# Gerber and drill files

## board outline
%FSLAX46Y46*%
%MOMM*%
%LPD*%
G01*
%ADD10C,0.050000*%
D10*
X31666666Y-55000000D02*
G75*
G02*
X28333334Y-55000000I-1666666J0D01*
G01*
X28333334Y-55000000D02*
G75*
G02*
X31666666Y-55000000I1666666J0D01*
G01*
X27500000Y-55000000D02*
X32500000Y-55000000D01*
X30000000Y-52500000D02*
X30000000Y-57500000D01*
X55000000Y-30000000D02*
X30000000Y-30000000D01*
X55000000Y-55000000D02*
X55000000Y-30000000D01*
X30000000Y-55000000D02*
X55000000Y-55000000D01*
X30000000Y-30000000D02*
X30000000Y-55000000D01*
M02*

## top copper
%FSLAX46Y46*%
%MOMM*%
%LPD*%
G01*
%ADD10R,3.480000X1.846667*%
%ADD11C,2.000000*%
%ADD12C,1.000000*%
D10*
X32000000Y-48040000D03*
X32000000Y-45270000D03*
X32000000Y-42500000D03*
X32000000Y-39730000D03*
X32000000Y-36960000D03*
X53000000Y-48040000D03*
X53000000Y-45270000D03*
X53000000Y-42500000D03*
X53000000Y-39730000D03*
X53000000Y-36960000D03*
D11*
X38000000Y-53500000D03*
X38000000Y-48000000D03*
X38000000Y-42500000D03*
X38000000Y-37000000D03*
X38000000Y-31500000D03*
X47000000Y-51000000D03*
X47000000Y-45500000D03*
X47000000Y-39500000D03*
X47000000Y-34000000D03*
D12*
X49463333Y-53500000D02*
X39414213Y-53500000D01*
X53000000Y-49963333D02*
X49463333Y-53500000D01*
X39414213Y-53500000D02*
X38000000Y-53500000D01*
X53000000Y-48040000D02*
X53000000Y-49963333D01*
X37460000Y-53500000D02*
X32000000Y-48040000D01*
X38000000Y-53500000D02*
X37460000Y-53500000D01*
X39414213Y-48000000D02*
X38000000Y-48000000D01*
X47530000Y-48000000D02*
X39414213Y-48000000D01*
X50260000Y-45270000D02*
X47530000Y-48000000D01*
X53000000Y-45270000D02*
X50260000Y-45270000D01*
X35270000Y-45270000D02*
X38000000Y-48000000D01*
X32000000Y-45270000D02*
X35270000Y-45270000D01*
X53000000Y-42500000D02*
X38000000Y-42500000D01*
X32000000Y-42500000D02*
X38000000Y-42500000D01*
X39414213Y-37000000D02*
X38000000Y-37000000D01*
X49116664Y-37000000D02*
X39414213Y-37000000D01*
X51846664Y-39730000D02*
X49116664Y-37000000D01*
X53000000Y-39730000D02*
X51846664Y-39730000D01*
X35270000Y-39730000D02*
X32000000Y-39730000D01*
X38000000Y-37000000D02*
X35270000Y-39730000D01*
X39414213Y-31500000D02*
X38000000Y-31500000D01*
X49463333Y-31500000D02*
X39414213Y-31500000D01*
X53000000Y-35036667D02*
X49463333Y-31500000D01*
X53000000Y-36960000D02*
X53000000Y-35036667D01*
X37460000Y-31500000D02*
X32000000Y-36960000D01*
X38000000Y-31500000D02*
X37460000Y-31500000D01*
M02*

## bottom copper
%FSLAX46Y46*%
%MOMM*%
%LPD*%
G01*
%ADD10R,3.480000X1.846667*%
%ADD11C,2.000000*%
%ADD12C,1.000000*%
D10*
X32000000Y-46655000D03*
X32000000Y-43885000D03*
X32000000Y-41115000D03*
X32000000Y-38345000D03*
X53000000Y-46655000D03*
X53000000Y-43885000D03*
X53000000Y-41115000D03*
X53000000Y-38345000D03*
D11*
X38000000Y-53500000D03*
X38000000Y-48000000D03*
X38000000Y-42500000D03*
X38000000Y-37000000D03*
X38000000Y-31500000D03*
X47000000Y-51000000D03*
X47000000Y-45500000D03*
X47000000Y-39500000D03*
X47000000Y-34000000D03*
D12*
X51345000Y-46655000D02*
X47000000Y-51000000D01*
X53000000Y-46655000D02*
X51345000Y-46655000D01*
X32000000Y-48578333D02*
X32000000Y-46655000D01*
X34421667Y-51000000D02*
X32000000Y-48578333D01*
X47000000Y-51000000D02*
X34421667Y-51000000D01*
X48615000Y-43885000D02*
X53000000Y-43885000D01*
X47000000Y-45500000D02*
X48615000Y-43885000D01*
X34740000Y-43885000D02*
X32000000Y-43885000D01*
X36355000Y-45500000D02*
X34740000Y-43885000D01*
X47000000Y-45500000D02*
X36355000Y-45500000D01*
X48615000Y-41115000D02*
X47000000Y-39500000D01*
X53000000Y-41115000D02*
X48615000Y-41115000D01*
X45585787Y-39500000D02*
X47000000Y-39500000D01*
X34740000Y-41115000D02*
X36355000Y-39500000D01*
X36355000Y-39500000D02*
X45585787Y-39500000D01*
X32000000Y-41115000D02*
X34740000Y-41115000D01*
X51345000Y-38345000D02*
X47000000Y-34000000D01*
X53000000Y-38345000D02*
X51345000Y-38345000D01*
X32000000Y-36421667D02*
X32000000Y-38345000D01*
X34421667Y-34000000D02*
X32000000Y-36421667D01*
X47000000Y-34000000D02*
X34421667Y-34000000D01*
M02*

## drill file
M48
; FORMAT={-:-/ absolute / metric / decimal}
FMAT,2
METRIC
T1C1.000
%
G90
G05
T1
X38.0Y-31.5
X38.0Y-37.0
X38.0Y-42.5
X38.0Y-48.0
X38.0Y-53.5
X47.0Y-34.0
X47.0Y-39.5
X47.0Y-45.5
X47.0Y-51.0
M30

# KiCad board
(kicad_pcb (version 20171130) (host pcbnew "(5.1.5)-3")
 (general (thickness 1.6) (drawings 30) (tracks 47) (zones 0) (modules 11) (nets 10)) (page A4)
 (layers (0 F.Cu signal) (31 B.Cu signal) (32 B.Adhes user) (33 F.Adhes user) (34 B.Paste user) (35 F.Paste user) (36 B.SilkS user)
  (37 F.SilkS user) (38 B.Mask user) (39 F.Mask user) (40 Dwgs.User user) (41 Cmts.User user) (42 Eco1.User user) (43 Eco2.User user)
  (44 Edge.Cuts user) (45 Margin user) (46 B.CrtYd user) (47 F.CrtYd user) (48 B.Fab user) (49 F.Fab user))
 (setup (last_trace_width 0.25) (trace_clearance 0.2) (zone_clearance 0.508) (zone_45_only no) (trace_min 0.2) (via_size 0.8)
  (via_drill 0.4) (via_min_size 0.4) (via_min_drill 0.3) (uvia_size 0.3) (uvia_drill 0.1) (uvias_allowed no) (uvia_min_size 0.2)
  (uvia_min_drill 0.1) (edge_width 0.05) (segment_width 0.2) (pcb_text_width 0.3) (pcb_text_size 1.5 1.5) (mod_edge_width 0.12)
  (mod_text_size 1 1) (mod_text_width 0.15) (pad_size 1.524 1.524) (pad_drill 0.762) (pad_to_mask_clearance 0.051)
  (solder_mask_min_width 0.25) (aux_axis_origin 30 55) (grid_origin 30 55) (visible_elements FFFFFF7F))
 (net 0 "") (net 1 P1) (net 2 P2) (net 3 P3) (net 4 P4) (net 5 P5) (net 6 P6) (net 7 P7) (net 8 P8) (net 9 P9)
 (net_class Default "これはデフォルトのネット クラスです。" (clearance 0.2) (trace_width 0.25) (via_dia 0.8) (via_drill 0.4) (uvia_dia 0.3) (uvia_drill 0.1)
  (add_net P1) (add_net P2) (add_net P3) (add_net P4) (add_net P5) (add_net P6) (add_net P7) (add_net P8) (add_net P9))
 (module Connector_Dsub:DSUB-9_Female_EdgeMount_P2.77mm (layer F.Cu) (at 32 42.5 270)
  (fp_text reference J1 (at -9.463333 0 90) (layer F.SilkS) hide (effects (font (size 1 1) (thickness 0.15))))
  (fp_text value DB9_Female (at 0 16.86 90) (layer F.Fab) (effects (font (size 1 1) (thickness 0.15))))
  (pad 1 smd rect (at 5.54 0 270) (size 1.846667 3.48) (layers F.Cu F.Paste F.Mask) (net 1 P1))
  (pad 2 smd rect (at 2.77 0 270) (size 1.846667 3.48) (layers F.Cu F.Paste F.Mask) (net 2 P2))
  (pad 3 smd rect (at 0 0 270) (size 1.846667 3.48) (layers F.Cu F.Paste F.Mask) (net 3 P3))
  (pad 4 smd rect (at -2.77 0 270) (size 1.846667 3.48) (layers F.Cu F.Paste F.Mask) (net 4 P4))
  (pad 5 smd rect (at -5.54 0 270) (size 1.846667 3.48) (layers F.Cu F.Paste F.Mask) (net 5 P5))
  (pad 6 smd rect (at 4.155 0 270) (size 1.846667 3.48) (layers B.Cu B.Paste B.Mask) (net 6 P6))
  (pad 7 smd rect (at 1.385 0 270) (size 1.846667 3.48) (layers B.Cu B.Paste B.Mask) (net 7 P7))
  (pad 8 smd rect (at -1.385 0 270) (size 1.846667 3.48) (layers B.Cu B.Paste B.Mask) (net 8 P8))
  (pad 9 smd rect (at -4.155 0 270) (size 1.846667 3.48) (layers B.Cu B.Paste B.Mask) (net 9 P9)))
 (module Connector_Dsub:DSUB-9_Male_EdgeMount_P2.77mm (layer F.Cu) (at 53 42.5 90)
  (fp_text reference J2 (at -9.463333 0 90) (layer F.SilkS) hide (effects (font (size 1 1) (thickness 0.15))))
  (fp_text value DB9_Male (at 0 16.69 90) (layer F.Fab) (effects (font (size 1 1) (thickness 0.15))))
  (pad 1 smd rect (at -5.54 0 90) (size 1.846667 3.48) (layers F.Cu F.Paste F.Mask) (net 1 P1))
  (pad 2 smd rect (at -2.77 0 90) (size 1.846667 3.48) (layers F.Cu F.Paste F.Mask) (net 2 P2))
  (pad 3 smd rect (at 0 0 90) (size 1.846667 3.48) (layers F.Cu F.Paste F.Mask) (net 3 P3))
  (pad 4 smd rect (at 2.77 0 90) (size 1.846667 3.48) (layers F.Cu F.Paste F.Mask) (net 4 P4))
  (pad 5 smd rect (at 5.54 0 90) (size 1.846667 3.48) (layers F.Cu F.Paste F.Mask) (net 5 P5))
  (pad 6 smd rect (at -4.155 0 90) (size 1.846667 3.48) (layers B.Cu B.Paste B.Mask) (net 6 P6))
  (pad 7 smd rect (at -1.385 0 90) (size 1.846667 3.48) (layers B.Cu B.Paste B.Mask) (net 7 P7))
  (pad 8 smd rect (at 1.385 0 90) (size 1.846667 3.48) (layers B.Cu B.Paste B.Mask) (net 8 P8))
  (pad 9 smd rect (at 4.155 0 90) (size 1.846667 3.48) (layers B.Cu B.Paste B.Mask) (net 9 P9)))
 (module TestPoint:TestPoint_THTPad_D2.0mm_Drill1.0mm (layer F.Cu) (at 38 53.5)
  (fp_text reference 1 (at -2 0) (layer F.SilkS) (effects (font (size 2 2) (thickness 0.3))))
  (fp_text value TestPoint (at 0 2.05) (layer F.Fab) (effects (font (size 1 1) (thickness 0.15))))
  (pad 1 thru_hole circle (at 0 0) (size 2 2) (drill 1) (layers *.Cu *.Mask) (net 1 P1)))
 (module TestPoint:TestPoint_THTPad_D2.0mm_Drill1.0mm (layer F.Cu) (at 38 48)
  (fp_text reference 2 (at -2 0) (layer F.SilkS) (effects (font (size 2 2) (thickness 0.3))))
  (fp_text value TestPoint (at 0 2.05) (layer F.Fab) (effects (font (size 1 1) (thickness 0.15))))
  (pad 1 thru_hole circle (at 0 0) (size 2 2) (drill 1) (layers *.Cu *.Mask) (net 2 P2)))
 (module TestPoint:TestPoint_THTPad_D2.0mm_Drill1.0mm (layer F.Cu) (at 38 42.5)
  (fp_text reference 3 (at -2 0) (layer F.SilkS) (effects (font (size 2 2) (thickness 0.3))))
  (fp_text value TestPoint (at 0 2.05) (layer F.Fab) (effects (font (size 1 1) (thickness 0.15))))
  (pad 1 thru_hole circle (at 0 0) (size 2 2) (drill 1) (layers *.Cu *.Mask) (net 3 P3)))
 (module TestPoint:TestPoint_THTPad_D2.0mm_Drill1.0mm (layer F.Cu) (at 38 37)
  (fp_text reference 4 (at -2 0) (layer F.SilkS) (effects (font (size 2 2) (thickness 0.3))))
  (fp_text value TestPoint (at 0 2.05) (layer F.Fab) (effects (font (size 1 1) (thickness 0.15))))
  (pad 1 thru_hole circle (at 0 0) (size 2 2) (drill 1) (layers *.Cu *.Mask) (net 4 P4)))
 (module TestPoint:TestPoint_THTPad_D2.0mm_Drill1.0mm (layer F.Cu) (at 38 31.5)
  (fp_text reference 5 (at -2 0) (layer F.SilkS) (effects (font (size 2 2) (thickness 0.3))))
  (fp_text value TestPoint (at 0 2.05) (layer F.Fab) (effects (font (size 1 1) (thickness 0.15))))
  (pad 1 thru_hole circle (at 0 0) (size 2 2) (drill 1) (layers *.Cu *.Mask) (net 5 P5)))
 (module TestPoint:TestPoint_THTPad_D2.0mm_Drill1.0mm (layer F.Cu) (at 47 51)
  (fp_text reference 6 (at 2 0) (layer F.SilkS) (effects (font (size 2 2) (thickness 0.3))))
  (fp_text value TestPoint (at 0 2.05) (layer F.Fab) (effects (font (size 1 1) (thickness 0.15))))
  (pad 1 thru_hole circle (at 0 0) (size 2 2) (drill 1) (layers *.Cu *.Mask) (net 6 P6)))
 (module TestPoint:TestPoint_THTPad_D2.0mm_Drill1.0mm (layer F.Cu) (at 47 45.5)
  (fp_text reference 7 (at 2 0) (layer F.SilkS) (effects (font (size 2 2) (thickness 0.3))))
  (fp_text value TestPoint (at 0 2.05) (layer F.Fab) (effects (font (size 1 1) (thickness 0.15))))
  (pad 1 thru_hole circle (at 0 0) (size 2 2) (drill 1) (layers *.Cu *.Mask) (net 7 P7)))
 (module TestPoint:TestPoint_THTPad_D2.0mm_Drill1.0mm (layer F.Cu) (at 47 39.5)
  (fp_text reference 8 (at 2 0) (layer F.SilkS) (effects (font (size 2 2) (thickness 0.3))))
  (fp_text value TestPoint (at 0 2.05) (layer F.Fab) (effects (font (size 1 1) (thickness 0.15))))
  (pad 1 thru_hole circle (at 0 0) (size 2 2) (drill 1) (layers *.Cu *.Mask) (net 8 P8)))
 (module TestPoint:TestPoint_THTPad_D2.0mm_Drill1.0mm (layer F.Cu) (at 47 34)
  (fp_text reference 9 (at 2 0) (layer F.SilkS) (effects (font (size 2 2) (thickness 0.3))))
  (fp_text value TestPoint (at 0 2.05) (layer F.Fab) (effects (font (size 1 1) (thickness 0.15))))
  (pad 1 thru_hole circle (at 0 0) (size 2 2) (drill 1) (layers *.Cu *.Mask) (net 9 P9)))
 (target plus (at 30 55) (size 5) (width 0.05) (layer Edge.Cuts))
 (gr_line (start 55 30) (end 30 30) (layer Edge.Cuts) (width 0.05))
 (gr_line (start 55 55) (end 55 30) (layer Edge.Cuts) (width 0.05))
 (gr_line (start 30 55) (end 55 55) (layer Edge.Cuts) (width 0.05))
 (gr_line (start 30 30) (end 30 55) (layer Edge.Cuts) (width 0.05))
 (segment (start 49.463333 53.5) (end 39.414213 53.5) (width 1) (layer F.Cu) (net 1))
 (segment (start 53 49.963333) (end 49.463333 53.5) (width 1) (layer F.Cu) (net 1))
 (segment (start 39.414213 53.5) (end 38 53.5) (width 1) (layer F.Cu) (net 1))
 (segment (start 53 48.04) (end 53 49.963333) (width 1) (layer F.Cu) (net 1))
 (segment (start 37.46 53.5) (end 32 48.04) (width 1) (layer F.Cu) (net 1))
 (segment (start 38 53.5) (end 37.46 53.5) (width 1) (layer F.Cu) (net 1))
 (segment (start 39.414213 48) (end 38 48) (width 1) (layer F.Cu) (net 2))
 (segment (start 47.53 48) (end 39.414213 48) (width 1) (layer F.Cu) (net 2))
 (segment (start 50.26 45.27) (end 47.53 48) (width 1) (layer F.Cu) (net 2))
 (segment (start 53 45.27) (end 50.26 45.27) (width 1) (layer F.Cu) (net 2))
 (segment (start 35.27 45.27) (end 38 48) (width 1) (layer F.Cu) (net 2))
 (segment (start 32 45.27) (end 35.27 45.27) (width 1) (layer F.Cu) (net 2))
 (segment (start 53 42.5) (end 38 42.5) (width 1) (layer F.Cu) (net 3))
 (segment (start 32 42.5) (end 38 42.5) (width 1) (layer F.Cu) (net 3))
 (segment (start 39.414213 37) (end 38 37) (width 1) (layer F.Cu) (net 4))
 (segment (start 49.116664 37) (end 39.414213 37) (width 1) (layer F.Cu) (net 4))
 (segment (start 51.846664 39.73) (end 49.116664 37) (width 1) (layer F.Cu) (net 4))
 (segment (start 53 39.73) (end 51.846664 39.73) (width 1) (layer F.Cu) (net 4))
 (segment (start 35.27 39.73) (end 32 39.73) (width 1) (layer F.Cu) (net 4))
 (segment (start 38 37) (end 35.27 39.73) (width 1) (layer F.Cu) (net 4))
 (segment (start 39.414213 31.5) (end 38 31.5) (width 1) (layer F.Cu) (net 5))
 (segment (start 49.463333 31.5) (end 39.414213 31.5) (width 1) (layer F.Cu) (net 5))
 (segment (start 53 35.036667) (end 49.463333 31.5) (width 1) (layer F.Cu) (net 5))
 (segment (start 53 36.96) (end 53 35.036667) (width 1) (layer F.Cu) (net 5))
 (segment (start 37.46 31.5) (end 32 36.96) (width 1) (layer F.Cu) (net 5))
 (segment (start 38 31.5) (end 37.46 31.5) (width 1) (layer F.Cu) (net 5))
 (segment (start 51.345 46.655) (end 47 51) (width 1) (layer B.Cu) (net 6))
 (segment (start 53 46.655) (end 51.345 46.655) (width 1) (layer B.Cu) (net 6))
 (segment (start 32 48.578333) (end 32 46.655) (width 1) (layer B.Cu) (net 6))
 (segment (start 34.421667 51) (end 32 48.578333) (width 1) (layer B.Cu) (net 6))
 (segment (start 47 51) (end 34.421667 51) (width 1) (layer B.Cu) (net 6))
 (segment (start 48.615 43.885) (end 53 43.885) (width 1) (layer B.Cu) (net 7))
 (segment (start 47 45.5) (end 48.615 43.885) (width 1) (layer B.Cu) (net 7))
 (segment (start 34.74 43.885) (end 32 43.885) (width 1) (layer B.Cu) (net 7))
 (segment (start 36.355 45.5) (end 34.74 43.885) (width 1) (layer B.Cu) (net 7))
 (segment (start 47 45.5) (end 36.355 45.5) (width 1) (layer B.Cu) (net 7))
 (segment (start 48.615 41.115) (end 47 39.5) (width 1) (layer B.Cu) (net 8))
 (segment (start 53 41.115) (end 48.615 41.115) (width 1) (layer B.Cu) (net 8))
 (segment (start 45.585787 39.5) (end 47 39.5) (width 1) (layer B.Cu) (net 8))
 (segment (start 34.74 41.115) (end 36.355 39.5) (width 1) (layer B.Cu) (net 8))
 (segment (start 36.355 39.5) (end 45.585787 39.5) (width 1) (layer B.Cu) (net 8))
 (segment (start 32 41.115) (end 34.74 41.115) (width 1) (layer B.Cu) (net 8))
 (segment (start 51.345 38.345) (end 47 34) (width 1) (layer B.Cu) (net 9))
 (segment (start 53 38.345) (end 51.345 38.345) (width 1) (layer B.Cu) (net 9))
 (segment (start 32 36.421667) (end 32 38.345) (width 1) (layer B.Cu) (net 9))
 (segment (start 34.421667 34) (end 32 36.421667) (width 1) (layer B.Cu) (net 9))
 (segment (start 47 34) (end 34.421667 34) (width 1) (layer B.Cu) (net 9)))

